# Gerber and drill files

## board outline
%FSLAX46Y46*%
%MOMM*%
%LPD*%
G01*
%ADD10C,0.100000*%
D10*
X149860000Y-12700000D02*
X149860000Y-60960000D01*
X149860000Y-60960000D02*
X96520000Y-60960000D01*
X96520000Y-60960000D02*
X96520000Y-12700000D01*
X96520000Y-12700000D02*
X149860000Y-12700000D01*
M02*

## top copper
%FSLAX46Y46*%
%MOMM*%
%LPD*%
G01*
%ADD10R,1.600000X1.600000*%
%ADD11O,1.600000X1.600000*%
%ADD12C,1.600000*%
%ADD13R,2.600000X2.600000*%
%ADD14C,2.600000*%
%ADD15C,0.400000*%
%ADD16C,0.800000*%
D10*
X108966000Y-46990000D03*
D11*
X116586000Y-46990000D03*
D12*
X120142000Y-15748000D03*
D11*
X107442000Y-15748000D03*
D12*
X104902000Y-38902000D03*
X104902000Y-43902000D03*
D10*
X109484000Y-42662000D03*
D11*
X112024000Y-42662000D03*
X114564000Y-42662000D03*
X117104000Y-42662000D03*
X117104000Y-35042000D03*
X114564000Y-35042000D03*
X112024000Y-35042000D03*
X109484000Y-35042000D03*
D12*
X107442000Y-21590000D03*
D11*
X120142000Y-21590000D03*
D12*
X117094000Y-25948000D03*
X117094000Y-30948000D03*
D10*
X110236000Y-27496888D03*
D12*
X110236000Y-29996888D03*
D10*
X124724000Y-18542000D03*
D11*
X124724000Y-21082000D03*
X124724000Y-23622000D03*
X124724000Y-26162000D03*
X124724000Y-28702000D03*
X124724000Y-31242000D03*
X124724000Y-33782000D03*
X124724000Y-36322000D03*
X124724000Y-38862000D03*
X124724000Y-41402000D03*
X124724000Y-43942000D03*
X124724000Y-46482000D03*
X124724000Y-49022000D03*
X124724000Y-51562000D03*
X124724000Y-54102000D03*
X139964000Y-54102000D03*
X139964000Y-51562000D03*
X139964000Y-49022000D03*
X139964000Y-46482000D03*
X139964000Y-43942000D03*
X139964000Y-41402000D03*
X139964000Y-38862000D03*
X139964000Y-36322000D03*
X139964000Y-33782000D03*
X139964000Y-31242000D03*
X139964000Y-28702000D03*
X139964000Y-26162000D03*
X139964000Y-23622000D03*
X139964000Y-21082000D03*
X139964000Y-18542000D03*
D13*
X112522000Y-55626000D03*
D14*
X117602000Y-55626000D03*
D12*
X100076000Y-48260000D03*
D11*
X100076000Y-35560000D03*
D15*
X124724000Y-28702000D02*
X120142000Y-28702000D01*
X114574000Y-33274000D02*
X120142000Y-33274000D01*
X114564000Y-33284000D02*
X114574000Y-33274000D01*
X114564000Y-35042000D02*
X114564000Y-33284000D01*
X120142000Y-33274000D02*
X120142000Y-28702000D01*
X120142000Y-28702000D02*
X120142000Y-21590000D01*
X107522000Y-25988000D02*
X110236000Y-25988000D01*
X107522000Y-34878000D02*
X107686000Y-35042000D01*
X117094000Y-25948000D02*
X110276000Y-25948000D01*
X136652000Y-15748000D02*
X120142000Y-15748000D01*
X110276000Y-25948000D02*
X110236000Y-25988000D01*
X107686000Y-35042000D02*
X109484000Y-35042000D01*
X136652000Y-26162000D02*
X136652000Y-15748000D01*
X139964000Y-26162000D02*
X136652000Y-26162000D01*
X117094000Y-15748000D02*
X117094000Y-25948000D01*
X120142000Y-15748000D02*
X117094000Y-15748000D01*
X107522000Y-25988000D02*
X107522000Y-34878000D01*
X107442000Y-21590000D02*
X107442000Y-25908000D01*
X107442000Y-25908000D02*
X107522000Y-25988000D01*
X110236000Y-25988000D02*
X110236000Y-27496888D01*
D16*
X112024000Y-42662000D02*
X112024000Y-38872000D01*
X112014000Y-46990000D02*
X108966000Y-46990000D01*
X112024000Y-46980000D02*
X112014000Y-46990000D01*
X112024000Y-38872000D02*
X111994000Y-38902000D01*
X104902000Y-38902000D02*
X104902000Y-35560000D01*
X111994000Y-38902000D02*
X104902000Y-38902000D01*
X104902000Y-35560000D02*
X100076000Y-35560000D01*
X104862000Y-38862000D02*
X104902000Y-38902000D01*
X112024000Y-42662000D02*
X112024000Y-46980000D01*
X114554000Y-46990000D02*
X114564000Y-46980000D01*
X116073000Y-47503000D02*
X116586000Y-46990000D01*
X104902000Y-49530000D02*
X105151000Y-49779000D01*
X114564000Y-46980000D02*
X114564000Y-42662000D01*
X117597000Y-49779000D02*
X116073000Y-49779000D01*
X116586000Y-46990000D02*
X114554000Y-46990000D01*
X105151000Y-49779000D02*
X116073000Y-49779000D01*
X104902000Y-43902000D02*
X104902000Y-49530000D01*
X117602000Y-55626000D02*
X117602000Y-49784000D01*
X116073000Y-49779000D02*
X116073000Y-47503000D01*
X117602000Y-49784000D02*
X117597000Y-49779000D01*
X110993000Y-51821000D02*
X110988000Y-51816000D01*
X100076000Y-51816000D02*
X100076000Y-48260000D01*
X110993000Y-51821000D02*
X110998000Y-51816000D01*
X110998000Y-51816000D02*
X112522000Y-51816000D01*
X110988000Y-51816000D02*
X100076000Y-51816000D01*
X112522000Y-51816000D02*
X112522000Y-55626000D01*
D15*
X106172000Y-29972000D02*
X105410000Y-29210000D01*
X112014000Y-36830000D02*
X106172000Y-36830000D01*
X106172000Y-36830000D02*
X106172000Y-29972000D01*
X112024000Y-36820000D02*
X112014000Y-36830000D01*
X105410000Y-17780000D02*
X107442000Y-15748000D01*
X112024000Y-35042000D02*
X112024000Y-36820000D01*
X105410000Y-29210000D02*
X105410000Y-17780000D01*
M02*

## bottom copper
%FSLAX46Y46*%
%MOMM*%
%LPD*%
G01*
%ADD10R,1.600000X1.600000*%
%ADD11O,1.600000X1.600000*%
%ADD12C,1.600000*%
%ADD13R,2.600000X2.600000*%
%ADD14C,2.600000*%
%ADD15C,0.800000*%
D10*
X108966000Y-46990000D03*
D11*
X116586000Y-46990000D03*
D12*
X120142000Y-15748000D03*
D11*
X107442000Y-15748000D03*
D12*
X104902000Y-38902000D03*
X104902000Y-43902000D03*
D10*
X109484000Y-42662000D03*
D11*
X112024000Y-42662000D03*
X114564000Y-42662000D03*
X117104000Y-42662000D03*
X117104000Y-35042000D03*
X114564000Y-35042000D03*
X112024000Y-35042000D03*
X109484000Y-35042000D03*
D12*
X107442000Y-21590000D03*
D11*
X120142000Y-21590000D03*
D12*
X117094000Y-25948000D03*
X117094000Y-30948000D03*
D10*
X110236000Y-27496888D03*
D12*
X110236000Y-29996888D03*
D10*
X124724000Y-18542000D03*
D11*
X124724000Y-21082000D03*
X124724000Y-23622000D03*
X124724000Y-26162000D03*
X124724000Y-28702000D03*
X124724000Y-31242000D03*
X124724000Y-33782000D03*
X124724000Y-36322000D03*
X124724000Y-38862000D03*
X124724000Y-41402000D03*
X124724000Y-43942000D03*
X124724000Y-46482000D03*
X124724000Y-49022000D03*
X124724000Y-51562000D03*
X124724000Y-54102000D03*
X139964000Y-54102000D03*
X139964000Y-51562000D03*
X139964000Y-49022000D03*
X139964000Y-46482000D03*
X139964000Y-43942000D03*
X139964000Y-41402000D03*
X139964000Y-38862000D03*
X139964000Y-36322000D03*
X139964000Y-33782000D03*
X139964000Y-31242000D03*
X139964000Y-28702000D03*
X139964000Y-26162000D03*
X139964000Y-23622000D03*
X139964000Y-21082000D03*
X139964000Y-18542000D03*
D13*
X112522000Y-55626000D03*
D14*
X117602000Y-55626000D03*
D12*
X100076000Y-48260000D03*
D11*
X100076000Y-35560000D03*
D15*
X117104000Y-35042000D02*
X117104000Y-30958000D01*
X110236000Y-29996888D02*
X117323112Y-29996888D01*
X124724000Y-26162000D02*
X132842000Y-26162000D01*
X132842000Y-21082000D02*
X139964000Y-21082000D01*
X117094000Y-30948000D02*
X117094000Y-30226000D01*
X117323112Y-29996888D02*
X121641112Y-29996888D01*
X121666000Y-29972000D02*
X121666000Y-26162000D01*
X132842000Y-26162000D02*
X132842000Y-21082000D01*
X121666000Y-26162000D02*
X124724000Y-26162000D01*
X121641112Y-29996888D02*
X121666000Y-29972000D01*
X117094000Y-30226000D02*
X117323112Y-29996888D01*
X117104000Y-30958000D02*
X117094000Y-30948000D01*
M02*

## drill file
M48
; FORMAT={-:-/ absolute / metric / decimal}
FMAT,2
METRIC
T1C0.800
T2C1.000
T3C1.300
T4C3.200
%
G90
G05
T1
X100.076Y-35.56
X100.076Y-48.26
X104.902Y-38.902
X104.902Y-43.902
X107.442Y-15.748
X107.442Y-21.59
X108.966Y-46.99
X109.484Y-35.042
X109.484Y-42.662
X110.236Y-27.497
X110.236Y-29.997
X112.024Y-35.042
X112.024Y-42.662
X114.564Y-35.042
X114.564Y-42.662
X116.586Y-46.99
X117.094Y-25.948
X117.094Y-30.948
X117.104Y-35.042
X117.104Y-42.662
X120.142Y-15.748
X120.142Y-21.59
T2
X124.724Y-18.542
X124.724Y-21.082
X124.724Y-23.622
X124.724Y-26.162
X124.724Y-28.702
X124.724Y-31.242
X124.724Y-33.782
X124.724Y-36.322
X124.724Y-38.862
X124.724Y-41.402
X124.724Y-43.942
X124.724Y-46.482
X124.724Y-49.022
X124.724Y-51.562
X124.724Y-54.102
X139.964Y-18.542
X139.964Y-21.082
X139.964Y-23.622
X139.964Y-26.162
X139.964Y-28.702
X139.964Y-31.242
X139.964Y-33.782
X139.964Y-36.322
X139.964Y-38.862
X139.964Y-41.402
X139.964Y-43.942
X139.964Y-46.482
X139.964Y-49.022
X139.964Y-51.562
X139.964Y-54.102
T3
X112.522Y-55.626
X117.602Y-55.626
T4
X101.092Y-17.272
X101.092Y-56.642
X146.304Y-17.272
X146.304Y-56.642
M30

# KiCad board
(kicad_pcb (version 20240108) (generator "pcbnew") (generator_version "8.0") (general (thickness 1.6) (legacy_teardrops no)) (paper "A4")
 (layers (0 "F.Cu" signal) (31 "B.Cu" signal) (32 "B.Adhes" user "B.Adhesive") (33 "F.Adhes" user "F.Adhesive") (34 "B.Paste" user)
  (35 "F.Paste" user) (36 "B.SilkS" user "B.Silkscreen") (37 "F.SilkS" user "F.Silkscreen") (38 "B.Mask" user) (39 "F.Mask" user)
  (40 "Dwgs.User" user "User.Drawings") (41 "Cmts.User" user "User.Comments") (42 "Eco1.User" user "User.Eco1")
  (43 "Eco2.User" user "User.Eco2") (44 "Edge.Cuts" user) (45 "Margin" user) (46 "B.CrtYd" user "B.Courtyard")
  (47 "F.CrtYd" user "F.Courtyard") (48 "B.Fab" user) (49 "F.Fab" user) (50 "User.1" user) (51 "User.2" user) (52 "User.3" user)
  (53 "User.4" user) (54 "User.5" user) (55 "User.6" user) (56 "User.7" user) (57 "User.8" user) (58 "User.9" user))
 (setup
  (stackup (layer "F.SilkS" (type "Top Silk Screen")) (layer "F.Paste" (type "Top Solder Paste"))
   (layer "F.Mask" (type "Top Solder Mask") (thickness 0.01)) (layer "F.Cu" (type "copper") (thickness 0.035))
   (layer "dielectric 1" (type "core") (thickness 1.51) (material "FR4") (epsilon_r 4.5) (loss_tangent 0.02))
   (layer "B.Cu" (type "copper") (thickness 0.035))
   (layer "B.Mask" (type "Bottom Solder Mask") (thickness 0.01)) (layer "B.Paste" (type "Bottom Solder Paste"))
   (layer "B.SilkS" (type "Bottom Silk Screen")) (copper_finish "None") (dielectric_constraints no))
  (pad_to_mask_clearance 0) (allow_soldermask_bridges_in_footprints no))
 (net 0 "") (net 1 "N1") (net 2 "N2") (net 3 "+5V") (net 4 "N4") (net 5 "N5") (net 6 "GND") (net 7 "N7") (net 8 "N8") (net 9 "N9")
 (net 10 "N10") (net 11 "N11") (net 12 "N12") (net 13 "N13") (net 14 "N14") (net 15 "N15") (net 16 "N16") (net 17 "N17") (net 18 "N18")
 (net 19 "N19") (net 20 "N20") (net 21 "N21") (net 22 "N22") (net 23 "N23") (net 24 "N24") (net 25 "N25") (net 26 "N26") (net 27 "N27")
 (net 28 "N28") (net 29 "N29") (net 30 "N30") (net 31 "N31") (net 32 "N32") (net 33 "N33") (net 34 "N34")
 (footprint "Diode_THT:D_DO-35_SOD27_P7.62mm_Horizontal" (layer "F.Cu") (at 108.966 46.99)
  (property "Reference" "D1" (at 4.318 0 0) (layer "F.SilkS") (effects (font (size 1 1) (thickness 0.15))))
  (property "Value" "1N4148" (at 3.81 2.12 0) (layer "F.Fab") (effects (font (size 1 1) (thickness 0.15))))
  (pad "1" thru_hole rect (at 0 0) (size 1.6 1.6) (drill 0.8) (layers "*.Cu" "*.Mask") (remove_unused_layers no) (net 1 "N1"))
  (pad "2" thru_hole oval (at 7.62 0) (size 1.6 1.6) (drill 0.8) (layers "*.Cu" "*.Mask") (remove_unused_layers no) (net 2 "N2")))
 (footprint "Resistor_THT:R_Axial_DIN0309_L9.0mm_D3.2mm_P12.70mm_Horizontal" (layer "F.Cu") (at 120.142 15.748 180)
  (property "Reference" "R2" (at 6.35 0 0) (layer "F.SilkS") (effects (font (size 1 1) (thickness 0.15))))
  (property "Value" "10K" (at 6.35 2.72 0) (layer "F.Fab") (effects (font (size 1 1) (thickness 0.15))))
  (pad "1" thru_hole circle (at 0 0 180) (size 1.6 1.6) (drill 0.8) (layers "*.Cu" "*.Mask") (remove_unused_layers no) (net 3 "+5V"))
  (pad "2" thru_hole oval (at 12.7 0 180) (size 1.6 1.6) (drill 0.8) (layers "*.Cu" "*.Mask") (remove_unused_layers no) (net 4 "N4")))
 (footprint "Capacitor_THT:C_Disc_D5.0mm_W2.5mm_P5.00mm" (layer "F.Cu") (at 104.902 38.902 -90)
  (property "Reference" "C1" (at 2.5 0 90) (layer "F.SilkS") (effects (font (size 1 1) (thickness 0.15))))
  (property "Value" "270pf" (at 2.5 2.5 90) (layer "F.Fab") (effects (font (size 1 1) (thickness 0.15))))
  (pad "1" thru_hole circle (at 0 0 270) (size 1.6 1.6) (drill 0.8) (layers "*.Cu" "*.Mask") (remove_unused_layers no) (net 1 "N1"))
  (pad "2" thru_hole circle (at 5 0 270) (size 1.6 1.6) (drill 0.8) (layers "*.Cu" "*.Mask") (remove_unused_layers no) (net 2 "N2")))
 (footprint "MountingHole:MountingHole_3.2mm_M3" (layer "F.Cu") (at 146.304 17.272)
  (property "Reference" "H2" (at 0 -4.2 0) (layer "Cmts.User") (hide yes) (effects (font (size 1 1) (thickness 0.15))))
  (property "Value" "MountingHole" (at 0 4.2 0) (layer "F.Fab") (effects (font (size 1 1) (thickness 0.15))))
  (pad "" np_thru_hole circle (at 0 0) (size 3.2 3.2) (drill 3.2) (layers "*.Cu" "*.Mask")))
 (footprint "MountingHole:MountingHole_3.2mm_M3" (layer "F.Cu") (at 101.092 17.272)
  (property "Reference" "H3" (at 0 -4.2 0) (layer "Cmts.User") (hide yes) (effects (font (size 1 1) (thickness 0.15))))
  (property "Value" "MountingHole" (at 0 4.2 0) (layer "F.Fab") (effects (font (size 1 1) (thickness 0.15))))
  (pad "" np_thru_hole circle (at 0 0) (size 3.2 3.2) (drill 3.2) (layers "*.Cu" "*.Mask")))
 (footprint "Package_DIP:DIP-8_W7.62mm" (layer "F.Cu") (at 109.484 42.662 90)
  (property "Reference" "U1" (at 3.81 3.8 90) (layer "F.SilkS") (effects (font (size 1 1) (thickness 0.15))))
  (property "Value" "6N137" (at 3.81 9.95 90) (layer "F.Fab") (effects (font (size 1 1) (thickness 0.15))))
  (pad "1" thru_hole rect (at 0 0 90) (size 1.6 1.6) (drill 0.8) (layers "*.Cu" "*.Mask") (remove_unused_layers no) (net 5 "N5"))
  (pad "2" thru_hole oval (at 0 2.54 90) (size 1.6 1.6) (drill 0.8) (layers "*.Cu" "*.Mask") (remove_unused_layers no) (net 1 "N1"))
  (pad "3" thru_hole oval (at 0 5.08 90) (size 1.6 1.6) (drill 0.8) (layers "*.Cu" "*.Mask") (remove_unused_layers no) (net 2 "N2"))
  (pad "4" thru_hole oval (at 0 7.62 90) (size 1.6 1.6) (drill 0.8) (layers "*.Cu" "*.Mask") (remove_unused_layers no))
  (pad "5" thru_hole oval (at 7.62 7.62 90) (size 1.6 1.6) (drill 0.8) (layers "*.Cu" "*.Mask") (remove_unused_layers no) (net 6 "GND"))
  (pad "6" thru_hole oval (at 7.62 5.08 90) (size 1.6 1.6) (drill 0.8) (layers "*.Cu" "*.Mask") (remove_unused_layers no) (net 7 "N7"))
  (pad "7" thru_hole oval (at 7.62 2.54 90) (size 1.6 1.6) (drill 0.8) (layers "*.Cu" "*.Mask") (remove_unused_layers no) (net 4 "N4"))
  (pad "8" thru_hole oval (at 7.62 0 90) (size 1.6 1.6) (drill 0.8) (layers "*.Cu" "*.Mask") (remove_unused_layers no) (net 3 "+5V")))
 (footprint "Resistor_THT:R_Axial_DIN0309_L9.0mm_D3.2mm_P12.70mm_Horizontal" (layer "F.Cu") (at 107.442 21.59)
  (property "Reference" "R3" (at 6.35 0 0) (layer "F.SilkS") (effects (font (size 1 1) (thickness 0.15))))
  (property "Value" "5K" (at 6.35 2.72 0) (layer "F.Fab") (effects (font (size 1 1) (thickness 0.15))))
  (pad "1" thru_hole circle (at 0 0) (size 1.6 1.6) (drill 0.8) (layers "*.Cu" "*.Mask") (remove_unused_layers no) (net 3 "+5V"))
  (pad "2" thru_hole oval (at 12.7 0) (size 1.6 1.6) (drill 0.8) (layers "*.Cu" "*.Mask") (remove_unused_layers no) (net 7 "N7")))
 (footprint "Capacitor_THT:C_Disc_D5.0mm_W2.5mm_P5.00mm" (layer "F.Cu") (at 117.094 25.948 -90)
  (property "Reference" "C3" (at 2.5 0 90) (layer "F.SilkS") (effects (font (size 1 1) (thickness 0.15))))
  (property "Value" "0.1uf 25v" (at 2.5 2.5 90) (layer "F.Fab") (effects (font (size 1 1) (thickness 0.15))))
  (pad "1" thru_hole circle (at 0 0 270) (size 1.6 1.6) (drill 0.8) (layers "*.Cu" "*.Mask") (remove_unused_layers no) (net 3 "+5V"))
  (pad "2" thru_hole circle (at 5 0 270) (size 1.6 1.6) (drill 0.8) (layers "*.Cu" "*.Mask") (remove_unused_layers no) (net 6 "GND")))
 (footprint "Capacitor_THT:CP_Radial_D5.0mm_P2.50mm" (layer "F.Cu") (at 110.236 27.496888 -90)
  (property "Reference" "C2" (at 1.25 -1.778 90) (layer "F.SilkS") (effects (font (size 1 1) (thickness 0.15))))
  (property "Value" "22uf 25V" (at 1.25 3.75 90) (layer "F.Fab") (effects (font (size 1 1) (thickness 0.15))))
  (pad "1" thru_hole rect (at 0 0 270) (size 1.6 1.6) (drill 0.8) (layers "*.Cu" "*.Mask") (remove_unused_layers no) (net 3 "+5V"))
  (pad "2" thru_hole circle (at 2.5 0 270) (size 1.6 1.6) (drill 0.8) (layers "*.Cu" "*.Mask") (remove_unused_layers no) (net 6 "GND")))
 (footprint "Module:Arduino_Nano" (layer "F.Cu") (at 124.724 18.542)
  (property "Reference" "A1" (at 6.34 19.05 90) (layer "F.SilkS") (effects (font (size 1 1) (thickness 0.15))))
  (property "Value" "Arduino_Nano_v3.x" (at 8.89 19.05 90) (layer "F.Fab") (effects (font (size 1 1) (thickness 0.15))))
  (pad "1" thru_hole rect (at 0 0) (size 1.6 1.6) (drill 1) (layers "*.Cu" "*.Mask") (remove_unused_layers no) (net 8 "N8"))
  (pad "2" thru_hole oval (at 0 2.54) (size 1.6 1.6) (drill 1) (layers "*.Cu" "*.Mask") (remove_unused_layers no) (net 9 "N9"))
  (pad "3" thru_hole oval (at 0 5.08) (size 1.6 1.6) (drill 1) (layers "*.Cu" "*.Mask") (remove_unused_layers no) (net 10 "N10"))
  (pad "4" thru_hole oval (at 0 7.62) (size 1.6 1.6) (drill 1) (layers "*.Cu" "*.Mask") (remove_unused_layers no) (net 6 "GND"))
  (pad "5" thru_hole oval (at 0 10.16) (size 1.6 1.6) (drill 1) (layers "*.Cu" "*.Mask") (remove_unused_layers no) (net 7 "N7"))
  (pad "6" thru_hole oval (at 0 12.7) (size 1.6 1.6) (drill 1) (layers "*.Cu" "*.Mask") (remove_unused_layers no) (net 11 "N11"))
  (pad "7" thru_hole oval (at 0 15.24) (size 1.6 1.6) (drill 1) (layers "*.Cu" "*.Mask") (remove_unused_layers no) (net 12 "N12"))
  (pad "8" thru_hole oval (at 0 17.78) (size 1.6 1.6) (drill 1) (layers "*.Cu" "*.Mask") (remove_unused_layers no) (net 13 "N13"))
  (pad "9" thru_hole oval (at 0 20.32) (size 1.6 1.6) (drill 1) (layers "*.Cu" "*.Mask") (remove_unused_layers no) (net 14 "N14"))
  (pad "10" thru_hole oval (at 0 22.86) (size 1.6 1.6) (drill 1) (layers "*.Cu" "*.Mask") (remove_unused_layers no) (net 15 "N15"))
  (pad "11" thru_hole oval (at 0 25.4) (size 1.6 1.6) (drill 1) (layers "*.Cu" "*.Mask") (remove_unused_layers no) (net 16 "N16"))
  (pad "12" thru_hole oval (at 0 27.94) (size 1.6 1.6) (drill 1) (layers "*.Cu" "*.Mask") (remove_unused_layers no) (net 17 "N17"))
  (pad "13" thru_hole oval (at 0 30.48) (size 1.6 1.6) (drill 1) (layers "*.Cu" "*.Mask") (remove_unused_layers no) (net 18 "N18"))
  (pad "14" thru_hole oval (at 0 33.02) (size 1.6 1.6) (drill 1) (layers "*.Cu" "*.Mask") (remove_unused_layers no) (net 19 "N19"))
  (pad "15" thru_hole oval (at 0 35.56) (size 1.6 1.6) (drill 1) (layers "*.Cu" "*.Mask") (remove_unused_layers no) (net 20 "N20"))
  (pad "16" thru_hole oval (at 15.24 35.56) (size 1.6 1.6) (drill 1) (layers "*.Cu" "*.Mask") (remove_unused_layers no) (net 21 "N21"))
  (pad "17" thru_hole oval (at 15.24 33.02) (size 1.6 1.6) (drill 1) (layers "*.Cu" "*.Mask") (remove_unused_layers no) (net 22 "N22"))
  (pad "18" thru_hole oval (at 15.24 30.48) (size 1.6 1.6) (drill 1) (layers "*.Cu" "*.Mask") (remove_unused_layers no) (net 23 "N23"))
  (pad "19" thru_hole oval (at 15.24 27.94) (size 1.6 1.6) (drill 1) (layers "*.Cu" "*.Mask") (remove_unused_layers no) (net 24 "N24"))
  (pad "20" thru_hole oval (at 15.24 25.4) (size 1.6 1.6) (drill 1) (layers "*.Cu" "*.Mask") (remove_unused_layers no) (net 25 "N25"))
  (pad "21" thru_hole oval (at 15.24 22.86) (size 1.6 1.6) (drill 1) (layers "*.Cu" "*.Mask") (remove_unused_layers no) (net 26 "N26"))
  (pad "22" thru_hole oval (at 15.24 20.32) (size 1.6 1.6) (drill 1) (layers "*.Cu" "*.Mask") (remove_unused_layers no) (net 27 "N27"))
  (pad "23" thru_hole oval (at 15.24 17.78) (size 1.6 1.6) (drill 1) (layers "*.Cu" "*.Mask") (remove_unused_layers no) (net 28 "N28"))
  (pad "24" thru_hole oval (at 15.24 15.24) (size 1.6 1.6) (drill 1) (layers "*.Cu" "*.Mask") (remove_unused_layers no) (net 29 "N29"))
  (pad "25" thru_hole oval (at 15.24 12.7) (size 1.6 1.6) (drill 1) (layers "*.Cu" "*.Mask") (remove_unused_layers no) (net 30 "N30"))
  (pad "26" thru_hole oval (at 15.24 10.16) (size 1.6 1.6) (drill 1) (layers "*.Cu" "*.Mask") (remove_unused_layers no) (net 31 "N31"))
  (pad "27" thru_hole oval (at 15.24 7.62) (size 1.6 1.6) (drill 1) (layers "*.Cu" "*.Mask") (remove_unused_layers no) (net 3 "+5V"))
  (pad "28" thru_hole oval (at 15.24 5.08) (size 1.6 1.6) (drill 1) (layers "*.Cu" "*.Mask") (remove_unused_layers no) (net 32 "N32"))
  (pad "29" thru_hole oval (at 15.24 2.54) (size 1.6 1.6) (drill 1) (layers "*.Cu" "*.Mask") (remove_unused_layers no) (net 6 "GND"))
  (pad "30" thru_hole oval (at 15.24 0) (size 1.6 1.6) (drill 1) (layers "*.Cu" "*.Mask") (remove_unused_layers no) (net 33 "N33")))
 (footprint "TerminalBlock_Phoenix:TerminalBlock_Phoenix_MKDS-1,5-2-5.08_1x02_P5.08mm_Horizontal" (layer "F.Cu") (at 112.522 55.626)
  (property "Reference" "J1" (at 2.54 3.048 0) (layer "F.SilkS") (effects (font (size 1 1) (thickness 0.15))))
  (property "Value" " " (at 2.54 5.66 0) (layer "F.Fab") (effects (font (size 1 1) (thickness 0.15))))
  (pad "1" thru_hole rect (at 0 0) (size 2.6 2.6) (drill 1.3) (layers "*.Cu" "*.Mask") (remove_unused_layers no) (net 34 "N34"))
  (pad "2" thru_hole circle (at 5.08 0) (size 2.6 2.6) (drill 1.3) (layers "*.Cu" "*.Mask") (remove_unused_layers no) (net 2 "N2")))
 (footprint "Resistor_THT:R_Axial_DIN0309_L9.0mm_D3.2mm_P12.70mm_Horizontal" (layer "F.Cu") (at 100.076 48.26 90)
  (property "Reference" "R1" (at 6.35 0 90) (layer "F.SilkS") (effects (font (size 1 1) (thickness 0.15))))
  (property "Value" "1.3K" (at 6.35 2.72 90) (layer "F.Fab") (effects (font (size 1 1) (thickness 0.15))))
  (pad "1" thru_hole circle (at 0 0 90) (size 1.6 1.6) (drill 0.8) (layers "*.Cu" "*.Mask") (remove_unused_layers no) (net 34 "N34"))
  (pad "2" thru_hole oval (at 12.7 0 90) (size 1.6 1.6) (drill 0.8) (layers "*.Cu" "*.Mask") (remove_unused_layers no) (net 1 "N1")))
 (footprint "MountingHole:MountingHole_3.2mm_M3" (layer "F.Cu") (at 101.092 56.642)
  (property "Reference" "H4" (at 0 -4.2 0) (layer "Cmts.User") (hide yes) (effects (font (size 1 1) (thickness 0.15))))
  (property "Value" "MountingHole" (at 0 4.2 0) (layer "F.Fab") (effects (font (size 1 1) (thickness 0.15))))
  (pad "" np_thru_hole circle (at 0 0) (size 3.2 3.2) (drill 3.2) (layers "*.Cu" "*.Mask")))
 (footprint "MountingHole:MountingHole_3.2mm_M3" (layer "F.Cu") (at 146.304 56.642)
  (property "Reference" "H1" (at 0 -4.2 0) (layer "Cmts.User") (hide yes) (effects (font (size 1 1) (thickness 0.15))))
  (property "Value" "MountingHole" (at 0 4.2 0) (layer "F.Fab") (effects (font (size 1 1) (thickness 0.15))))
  (pad "" np_thru_hole circle (at 0 0) (size 3.2 3.2) (drill 3.2) (layers "*.Cu" "*.Mask")))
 (gr_line (start 149.86 12.7) (end 149.86 60.96) (stroke (width 0.1) (type solid)) (layer "Edge.Cuts"))
 (gr_line (start 149.86 60.96) (end 96.52 60.96) (stroke (width 0.1) (type solid)) (layer "Edge.Cuts"))
 (gr_line (start 96.52 60.96) (end 96.52 12.7) (stroke (width 0.1) (type solid)) (layer "Edge.Cuts"))
 (gr_line (start 96.52 12.7) (end 149.86 12.7) (stroke (width 0.1) (type solid)) (layer "Edge.Cuts"))
 (segment (start 117.104 35.042) (end 117.104 30.958) (width 0.8) (layer "B.Cu") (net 6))
 (segment (start 110.236 29.996888) (end 117.323112 29.996888) (width 0.8) (layer "B.Cu") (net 6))
 (segment (start 124.724 26.162) (end 132.842 26.162) (width 0.8) (layer "B.Cu") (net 6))
 (segment (start 132.842 21.082) (end 139.964 21.082) (width 0.8) (layer "B.Cu") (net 6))
 (segment (start 117.094 30.948) (end 117.094 30.226) (width 0.8) (layer "B.Cu") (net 6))
 (segment (start 117.323112 29.996888) (end 121.641112 29.996888) (width 0.8) (layer "B.Cu") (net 6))
 (segment (start 121.666 29.972) (end 121.666 26.162) (width 0.8) (layer "B.Cu") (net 6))
 (segment (start 132.842 26.162) (end 132.842 21.082) (width 0.8) (layer "B.Cu") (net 6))
 (segment (start 121.666 26.162) (end 124.724 26.162) (width 0.8) (layer "B.Cu") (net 6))
 (segment (start 121.641112 29.996888) (end 121.666 29.972) (width 0.8) (layer "B.Cu") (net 6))
 (segment (start 117.094 30.226) (end 117.323112 29.996888) (width 0.8) (layer "B.Cu") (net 6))
 (segment (start 117.104 30.958) (end 117.094 30.948) (width 0.8) (layer "B.Cu") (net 6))
 (segment (start 124.724 28.702) (end 120.142 28.702) (width 0.4) (layer "F.Cu") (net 7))
 (segment (start 114.574 33.274) (end 120.142 33.274) (width 0.4) (layer "F.Cu") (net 7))
 (segment (start 114.564 33.284) (end 114.574 33.274) (width 0.4) (layer "F.Cu") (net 7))
 (segment (start 114.564 35.042) (end 114.564 33.284) (width 0.4) (layer "F.Cu") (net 7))
 (segment (start 120.142 33.274) (end 120.142 28.702) (width 0.4) (layer "F.Cu") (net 7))
 (segment (start 120.142 28.702) (end 120.142 21.59) (width 0.4) (layer "F.Cu") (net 7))
 (segment (start 107.522 25.988) (end 110.236 25.988) (width 0.4) (layer "F.Cu") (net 3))
 (segment (start 107.522 34.878) (end 107.686 35.042) (width 0.4) (layer "F.Cu") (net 3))
 (segment (start 117.094 25.948) (end 110.276 25.948) (width 0.4) (layer "F.Cu") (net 3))
 (segment (start 136.652 15.748) (end 120.142 15.748) (width 0.4) (layer "F.Cu") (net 3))
 (segment (start 110.276 25.948) (end 110.236 25.988) (width 0.4) (layer "F.Cu") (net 3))
 (segment (start 107.686 35.042) (end 109.484 35.042) (width 0.4) (layer "F.Cu") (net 3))
 (segment (start 136.652 26.162) (end 136.652 15.748) (width 0.4) (layer "F.Cu") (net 3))
 (segment (start 139.964 26.162) (end 136.652 26.162) (width 0.4) (layer "F.Cu") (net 3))
 (segment (start 117.094 15.748) (end 117.094 25.948) (width 0.4) (layer "F.Cu") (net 3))
 (segment (start 120.142 15.748) (end 117.094 15.748) (width 0.4) (layer "F.Cu") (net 3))
 (segment (start 107.522 25.988) (end 107.522 34.878) (width 0.4) (layer "F.Cu") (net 3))
 (segment (start 107.442 21.59) (end 107.442 25.908) (width 0.4) (layer "F.Cu") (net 3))
 (segment (start 107.442 25.908) (end 107.522 25.988) (width 0.4) (layer "F.Cu") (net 3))
 (segment (start 110.236 25.988) (end 110.236 27.496888) (width 0.4) (layer "F.Cu") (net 3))
 (segment (start 112.024 42.662) (end 112.024 38.872) (width 0.8) (layer "F.Cu") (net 1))
 (segment (start 112.014 46.99) (end 108.966 46.99) (width 0.8) (layer "F.Cu") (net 1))
 (segment (start 112.024 46.98) (end 112.014 46.99) (width 0.8) (layer "F.Cu") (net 1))
 (segment (start 112.024 38.872) (end 111.994 38.902) (width 0.8) (layer "F.Cu") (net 1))
 (segment (start 104.902 38.902) (end 104.902 35.56) (width 0.8) (layer "F.Cu") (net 1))
 (segment (start 111.994 38.902) (end 104.902 38.902) (width 0.8) (layer "F.Cu") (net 1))
 (segment (start 104.902 35.56) (end 100.076 35.56) (width 0.8) (layer "F.Cu") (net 1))
 (segment (start 104.862 38.862) (end 104.902 38.902) (width 0.8) (layer "F.Cu") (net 1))
 (segment (start 112.024 42.662) (end 112.024 46.98) (width 0.8) (layer "F.Cu") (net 1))
 (segment (start 114.554 46.99) (end 114.564 46.98) (width 0.8) (layer "F.Cu") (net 2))
 (segment (start 116.073 47.503) (end 116.586 46.99) (width 0.8) (layer "F.Cu") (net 2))
 (segment (start 104.902 49.53) (end 105.151 49.779) (width 0.8) (layer "F.Cu") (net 2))
 (segment (start 114.564 46.98) (end 114.564 42.662) (width 0.8) (layer "F.Cu") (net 2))
 (segment (start 117.597 49.779) (end 116.073 49.779) (width 0.8) (layer "F.Cu") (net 2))
 (segment (start 116.586 46.99) (end 114.554 46.99) (width 0.8) (layer "F.Cu") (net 2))
 (segment (start 105.151 49.779) (end 116.073 49.779) (width 0.8) (layer "F.Cu") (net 2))
 (segment (start 104.902 43.902) (end 104.902 49.53) (width 0.8) (layer "F.Cu") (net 2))
 (segment (start 117.602 55.626) (end 117.602 49.784) (width 0.8) (layer "F.Cu") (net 2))
 (segment (start 116.073 49.779) (end 116.073 47.503) (width 0.8) (layer "F.Cu") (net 2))
 (segment (start 117.602 49.784) (end 117.597 49.779) (width 0.8) (layer "F.Cu") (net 2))
 (segment (start 110.993 51.821) (end 110.988 51.816) (width 0.8) (layer "F.Cu") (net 34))
 (segment (start 100.076 51.816) (end 100.076 48.26) (width 0.8) (layer "F.Cu") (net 34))
 (segment (start 110.993 51.821) (end 110.998 51.816) (width 0.8) (layer "F.Cu") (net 34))
 (segment (start 110.998 51.816) (end 112.522 51.816) (width 0.8) (layer "F.Cu") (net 34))
 (segment (start 110.988 51.816) (end 100.076 51.816) (width 0.8) (layer "F.Cu") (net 34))
 (segment (start 112.522 51.816) (end 112.522 55.626) (width 0.8) (layer "F.Cu") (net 34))
 (segment (start 106.172 29.972) (end 105.41 29.21) (width 0.4) (layer "F.Cu") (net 4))
 (segment (start 112.014 36.83) (end 106.172 36.83) (width 0.4) (layer "F.Cu") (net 4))
 (segment (start 106.172 36.83) (end 106.172 29.972) (width 0.4) (layer "F.Cu") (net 4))
 (segment (start 112.024 36.82) (end 112.014 36.83) (width 0.4) (layer "F.Cu") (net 4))
 (segment (start 105.41 17.78) (end 107.442 15.748) (width 0.4) (layer "F.Cu") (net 4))
 (segment (start 112.024 35.042) (end 112.024 36.82) (width 0.4) (layer "F.Cu") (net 4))
 (segment (start 105.41 29.21) (end 105.41 17.78) (width 0.4) (layer "F.Cu") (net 4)))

